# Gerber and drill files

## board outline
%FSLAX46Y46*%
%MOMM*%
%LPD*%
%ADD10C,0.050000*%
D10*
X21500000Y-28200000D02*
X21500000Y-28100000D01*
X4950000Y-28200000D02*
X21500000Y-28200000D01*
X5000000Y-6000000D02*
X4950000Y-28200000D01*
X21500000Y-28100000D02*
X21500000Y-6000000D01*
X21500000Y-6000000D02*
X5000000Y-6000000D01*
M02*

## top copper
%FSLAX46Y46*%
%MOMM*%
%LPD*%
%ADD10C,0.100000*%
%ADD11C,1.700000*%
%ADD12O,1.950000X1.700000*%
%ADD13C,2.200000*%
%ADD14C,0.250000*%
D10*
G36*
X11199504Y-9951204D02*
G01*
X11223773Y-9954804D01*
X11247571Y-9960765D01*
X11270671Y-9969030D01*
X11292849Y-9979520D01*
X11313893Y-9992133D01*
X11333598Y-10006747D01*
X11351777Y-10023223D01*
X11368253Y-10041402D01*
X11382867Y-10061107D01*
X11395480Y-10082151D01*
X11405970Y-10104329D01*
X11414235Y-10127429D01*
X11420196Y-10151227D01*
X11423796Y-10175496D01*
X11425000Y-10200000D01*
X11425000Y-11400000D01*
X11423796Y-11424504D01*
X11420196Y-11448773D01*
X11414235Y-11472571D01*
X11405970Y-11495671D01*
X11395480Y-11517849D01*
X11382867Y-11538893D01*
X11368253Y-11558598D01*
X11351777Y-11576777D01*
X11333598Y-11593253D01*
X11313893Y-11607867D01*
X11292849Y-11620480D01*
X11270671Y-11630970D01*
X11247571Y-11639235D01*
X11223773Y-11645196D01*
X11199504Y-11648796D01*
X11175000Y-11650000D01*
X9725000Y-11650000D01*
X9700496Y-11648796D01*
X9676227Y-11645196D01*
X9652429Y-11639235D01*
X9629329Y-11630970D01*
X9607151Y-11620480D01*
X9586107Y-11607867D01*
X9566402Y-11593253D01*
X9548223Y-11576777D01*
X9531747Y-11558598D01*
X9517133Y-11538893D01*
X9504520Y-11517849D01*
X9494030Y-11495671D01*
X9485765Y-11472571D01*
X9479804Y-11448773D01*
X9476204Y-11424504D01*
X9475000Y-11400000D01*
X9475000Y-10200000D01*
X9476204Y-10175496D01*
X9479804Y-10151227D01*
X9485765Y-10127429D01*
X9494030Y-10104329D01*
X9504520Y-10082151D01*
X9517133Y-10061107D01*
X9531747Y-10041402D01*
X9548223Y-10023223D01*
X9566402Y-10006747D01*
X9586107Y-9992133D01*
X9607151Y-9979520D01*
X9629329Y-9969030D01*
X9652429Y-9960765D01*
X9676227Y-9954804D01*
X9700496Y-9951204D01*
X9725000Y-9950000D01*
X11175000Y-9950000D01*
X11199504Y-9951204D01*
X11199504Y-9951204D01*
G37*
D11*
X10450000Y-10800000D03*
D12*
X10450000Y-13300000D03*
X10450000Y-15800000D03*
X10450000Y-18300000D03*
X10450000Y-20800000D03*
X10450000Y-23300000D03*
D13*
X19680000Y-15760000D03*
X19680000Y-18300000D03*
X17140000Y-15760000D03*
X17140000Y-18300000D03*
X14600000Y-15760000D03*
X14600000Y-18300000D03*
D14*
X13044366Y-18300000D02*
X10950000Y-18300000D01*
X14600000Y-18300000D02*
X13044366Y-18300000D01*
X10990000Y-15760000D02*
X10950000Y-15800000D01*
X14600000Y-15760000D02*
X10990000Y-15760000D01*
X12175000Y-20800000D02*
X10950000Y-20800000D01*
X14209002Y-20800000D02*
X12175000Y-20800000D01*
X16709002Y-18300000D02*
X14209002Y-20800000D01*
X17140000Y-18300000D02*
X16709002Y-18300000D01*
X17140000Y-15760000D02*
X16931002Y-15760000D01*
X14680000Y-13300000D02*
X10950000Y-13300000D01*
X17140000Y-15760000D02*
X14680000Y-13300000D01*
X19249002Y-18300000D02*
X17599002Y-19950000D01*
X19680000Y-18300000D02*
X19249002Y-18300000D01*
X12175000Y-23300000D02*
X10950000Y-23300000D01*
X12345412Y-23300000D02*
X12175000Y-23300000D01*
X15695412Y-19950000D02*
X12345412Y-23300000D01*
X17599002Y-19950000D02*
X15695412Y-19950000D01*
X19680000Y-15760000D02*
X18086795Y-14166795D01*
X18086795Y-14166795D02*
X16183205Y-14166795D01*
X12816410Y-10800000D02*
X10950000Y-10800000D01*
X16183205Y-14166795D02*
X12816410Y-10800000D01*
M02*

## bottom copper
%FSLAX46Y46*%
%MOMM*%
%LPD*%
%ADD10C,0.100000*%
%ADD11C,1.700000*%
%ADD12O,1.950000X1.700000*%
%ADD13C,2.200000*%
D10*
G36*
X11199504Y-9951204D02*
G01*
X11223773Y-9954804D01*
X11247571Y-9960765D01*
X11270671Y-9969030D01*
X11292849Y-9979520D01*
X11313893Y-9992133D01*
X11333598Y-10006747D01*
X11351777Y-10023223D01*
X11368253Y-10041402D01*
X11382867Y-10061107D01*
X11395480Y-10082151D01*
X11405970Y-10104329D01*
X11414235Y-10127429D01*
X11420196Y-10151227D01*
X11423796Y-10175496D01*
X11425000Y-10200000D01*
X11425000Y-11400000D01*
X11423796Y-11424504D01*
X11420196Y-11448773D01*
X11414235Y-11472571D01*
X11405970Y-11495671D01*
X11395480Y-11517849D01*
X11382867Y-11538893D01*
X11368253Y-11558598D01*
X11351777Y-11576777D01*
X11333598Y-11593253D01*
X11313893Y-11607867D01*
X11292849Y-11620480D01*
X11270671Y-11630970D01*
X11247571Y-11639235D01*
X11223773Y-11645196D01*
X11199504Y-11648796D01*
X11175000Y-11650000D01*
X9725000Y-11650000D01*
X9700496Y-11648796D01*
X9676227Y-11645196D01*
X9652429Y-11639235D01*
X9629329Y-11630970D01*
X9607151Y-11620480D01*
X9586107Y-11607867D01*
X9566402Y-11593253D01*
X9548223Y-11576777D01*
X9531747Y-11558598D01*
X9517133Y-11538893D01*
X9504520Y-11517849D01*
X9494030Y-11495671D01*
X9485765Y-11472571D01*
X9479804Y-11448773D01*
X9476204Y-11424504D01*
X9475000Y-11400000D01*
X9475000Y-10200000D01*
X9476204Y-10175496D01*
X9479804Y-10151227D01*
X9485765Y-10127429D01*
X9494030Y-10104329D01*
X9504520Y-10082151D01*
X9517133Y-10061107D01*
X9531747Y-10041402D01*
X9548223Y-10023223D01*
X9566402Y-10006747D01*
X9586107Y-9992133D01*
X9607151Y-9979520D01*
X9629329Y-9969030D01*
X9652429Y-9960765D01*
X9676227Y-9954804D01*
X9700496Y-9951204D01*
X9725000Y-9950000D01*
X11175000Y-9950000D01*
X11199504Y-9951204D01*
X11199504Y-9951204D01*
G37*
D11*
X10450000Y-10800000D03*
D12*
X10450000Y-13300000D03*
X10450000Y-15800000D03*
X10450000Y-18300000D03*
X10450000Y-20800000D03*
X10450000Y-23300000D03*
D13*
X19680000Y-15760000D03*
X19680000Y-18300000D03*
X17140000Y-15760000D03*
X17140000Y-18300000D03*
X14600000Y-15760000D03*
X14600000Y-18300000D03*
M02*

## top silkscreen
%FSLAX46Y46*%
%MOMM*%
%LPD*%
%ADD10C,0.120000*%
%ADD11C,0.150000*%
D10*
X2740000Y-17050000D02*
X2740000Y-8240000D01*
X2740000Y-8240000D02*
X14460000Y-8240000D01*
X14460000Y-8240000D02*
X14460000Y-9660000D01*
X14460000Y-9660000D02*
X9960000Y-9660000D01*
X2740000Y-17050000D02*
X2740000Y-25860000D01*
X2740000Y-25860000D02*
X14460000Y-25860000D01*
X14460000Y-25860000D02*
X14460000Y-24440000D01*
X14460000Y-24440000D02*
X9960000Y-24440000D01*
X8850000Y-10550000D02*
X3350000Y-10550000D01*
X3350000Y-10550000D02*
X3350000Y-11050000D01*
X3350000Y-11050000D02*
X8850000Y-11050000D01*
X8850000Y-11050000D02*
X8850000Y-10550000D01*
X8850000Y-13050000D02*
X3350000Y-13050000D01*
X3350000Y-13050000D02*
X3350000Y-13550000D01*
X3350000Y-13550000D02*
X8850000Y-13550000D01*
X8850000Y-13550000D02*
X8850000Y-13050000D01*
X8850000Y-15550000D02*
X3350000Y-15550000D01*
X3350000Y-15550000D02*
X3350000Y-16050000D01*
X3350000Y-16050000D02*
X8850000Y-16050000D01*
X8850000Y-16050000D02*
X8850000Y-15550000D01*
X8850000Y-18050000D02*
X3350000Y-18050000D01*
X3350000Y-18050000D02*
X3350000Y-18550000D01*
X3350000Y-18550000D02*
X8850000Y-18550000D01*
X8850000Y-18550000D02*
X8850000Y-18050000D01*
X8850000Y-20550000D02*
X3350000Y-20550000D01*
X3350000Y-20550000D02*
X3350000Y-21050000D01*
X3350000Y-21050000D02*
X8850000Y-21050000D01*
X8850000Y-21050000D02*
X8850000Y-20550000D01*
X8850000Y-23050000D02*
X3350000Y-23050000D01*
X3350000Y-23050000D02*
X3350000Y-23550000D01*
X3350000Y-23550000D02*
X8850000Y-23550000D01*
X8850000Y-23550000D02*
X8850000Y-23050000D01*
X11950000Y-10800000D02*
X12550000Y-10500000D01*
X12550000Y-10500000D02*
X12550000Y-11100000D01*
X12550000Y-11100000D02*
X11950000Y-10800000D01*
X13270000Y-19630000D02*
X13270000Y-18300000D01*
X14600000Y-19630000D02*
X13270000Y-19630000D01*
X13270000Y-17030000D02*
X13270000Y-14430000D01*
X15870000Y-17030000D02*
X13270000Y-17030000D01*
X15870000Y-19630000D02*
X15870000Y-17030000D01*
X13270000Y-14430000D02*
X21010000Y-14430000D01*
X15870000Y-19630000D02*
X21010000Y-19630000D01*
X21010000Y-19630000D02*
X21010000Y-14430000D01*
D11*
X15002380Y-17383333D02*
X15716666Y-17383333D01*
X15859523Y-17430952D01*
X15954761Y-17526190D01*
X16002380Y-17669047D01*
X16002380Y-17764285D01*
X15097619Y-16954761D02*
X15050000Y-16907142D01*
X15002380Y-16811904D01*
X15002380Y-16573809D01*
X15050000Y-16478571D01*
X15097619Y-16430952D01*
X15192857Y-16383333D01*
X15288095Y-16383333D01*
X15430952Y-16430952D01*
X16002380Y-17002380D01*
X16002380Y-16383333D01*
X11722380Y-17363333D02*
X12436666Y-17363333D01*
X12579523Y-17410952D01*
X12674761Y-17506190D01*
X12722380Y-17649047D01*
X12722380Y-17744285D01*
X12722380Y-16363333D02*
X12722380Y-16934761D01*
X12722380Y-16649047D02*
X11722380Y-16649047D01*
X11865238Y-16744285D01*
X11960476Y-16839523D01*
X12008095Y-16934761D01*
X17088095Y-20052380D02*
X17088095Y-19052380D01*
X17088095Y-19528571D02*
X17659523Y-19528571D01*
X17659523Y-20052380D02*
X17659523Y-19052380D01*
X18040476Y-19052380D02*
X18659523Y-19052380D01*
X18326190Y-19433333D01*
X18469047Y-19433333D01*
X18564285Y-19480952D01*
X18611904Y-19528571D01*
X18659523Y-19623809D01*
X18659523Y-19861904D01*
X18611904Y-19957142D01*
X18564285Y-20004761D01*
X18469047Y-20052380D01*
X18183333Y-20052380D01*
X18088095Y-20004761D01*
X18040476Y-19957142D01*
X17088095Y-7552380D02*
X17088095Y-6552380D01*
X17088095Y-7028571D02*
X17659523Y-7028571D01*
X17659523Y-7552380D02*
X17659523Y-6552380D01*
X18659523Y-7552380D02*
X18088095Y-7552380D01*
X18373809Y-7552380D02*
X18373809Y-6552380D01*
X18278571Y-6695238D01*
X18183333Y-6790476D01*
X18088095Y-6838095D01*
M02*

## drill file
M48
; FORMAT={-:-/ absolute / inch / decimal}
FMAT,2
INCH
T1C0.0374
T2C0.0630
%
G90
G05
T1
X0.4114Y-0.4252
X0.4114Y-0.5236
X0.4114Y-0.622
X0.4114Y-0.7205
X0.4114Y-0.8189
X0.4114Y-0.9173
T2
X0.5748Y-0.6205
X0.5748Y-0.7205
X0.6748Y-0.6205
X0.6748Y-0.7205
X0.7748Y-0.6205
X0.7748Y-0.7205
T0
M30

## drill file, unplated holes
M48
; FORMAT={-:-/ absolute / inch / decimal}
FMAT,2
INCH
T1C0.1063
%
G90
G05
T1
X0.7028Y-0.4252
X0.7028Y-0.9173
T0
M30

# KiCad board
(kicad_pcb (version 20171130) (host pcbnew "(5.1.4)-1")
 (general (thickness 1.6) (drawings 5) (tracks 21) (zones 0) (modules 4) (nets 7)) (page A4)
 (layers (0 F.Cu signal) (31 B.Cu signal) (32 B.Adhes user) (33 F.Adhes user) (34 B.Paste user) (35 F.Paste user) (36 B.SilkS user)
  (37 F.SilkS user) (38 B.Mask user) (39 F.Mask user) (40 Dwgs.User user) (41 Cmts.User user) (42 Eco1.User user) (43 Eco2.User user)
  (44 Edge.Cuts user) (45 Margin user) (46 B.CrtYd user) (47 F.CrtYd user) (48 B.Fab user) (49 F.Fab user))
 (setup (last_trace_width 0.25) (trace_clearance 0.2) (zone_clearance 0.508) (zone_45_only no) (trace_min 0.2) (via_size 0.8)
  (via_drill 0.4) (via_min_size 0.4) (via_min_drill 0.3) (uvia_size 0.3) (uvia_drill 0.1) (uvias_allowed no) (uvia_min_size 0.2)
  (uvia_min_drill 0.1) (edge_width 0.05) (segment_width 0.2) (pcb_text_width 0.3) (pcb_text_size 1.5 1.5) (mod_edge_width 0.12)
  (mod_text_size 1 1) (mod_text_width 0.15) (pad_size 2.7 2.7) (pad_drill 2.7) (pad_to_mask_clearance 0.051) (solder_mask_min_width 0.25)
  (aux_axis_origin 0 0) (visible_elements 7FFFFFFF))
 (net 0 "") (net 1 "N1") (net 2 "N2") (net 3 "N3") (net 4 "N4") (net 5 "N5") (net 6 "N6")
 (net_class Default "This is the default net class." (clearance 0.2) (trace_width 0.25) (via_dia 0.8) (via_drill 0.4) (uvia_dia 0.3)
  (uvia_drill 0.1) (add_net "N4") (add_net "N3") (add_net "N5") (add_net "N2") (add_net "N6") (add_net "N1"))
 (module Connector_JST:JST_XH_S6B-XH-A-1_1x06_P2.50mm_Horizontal (layer F.Cu) (at 10.45 10.8 270)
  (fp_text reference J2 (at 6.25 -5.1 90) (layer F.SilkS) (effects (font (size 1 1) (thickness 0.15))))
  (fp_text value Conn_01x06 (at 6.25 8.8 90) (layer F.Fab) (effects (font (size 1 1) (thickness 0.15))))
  (fp_line (start 6.25 7.71) (end -2.56 7.71) (layer F.SilkS) (width 0.12))
  (fp_line (start -2.56 7.71) (end -2.56 -4.01) (layer F.SilkS) (width 0.12))
  (fp_line (start -2.56 -4.01) (end -1.14 -4.01) (layer F.SilkS) (width 0.12))
  (fp_line (start -1.14 -4.01) (end -1.14 0.49) (layer F.SilkS) (width 0.12))
  (fp_line (start 6.25 7.71) (end 15.06 7.71) (layer F.SilkS) (width 0.12))
  (fp_line (start 15.06 7.71) (end 15.06 -4.01) (layer F.SilkS) (width 0.12))
  (fp_line (start 15.06 -4.01) (end 13.64 -4.01) (layer F.SilkS) (width 0.12))
  (fp_line (start 13.64 -4.01) (end 13.64 0.49) (layer F.SilkS) (width 0.12))
  (fp_line (start -0.25 1.6) (end -0.25 7.1) (layer F.SilkS) (width 0.12))
  (fp_line (start -0.25 7.1) (end 0.25 7.1) (layer F.SilkS) (width 0.12))
  (fp_line (start 0.25 7.1) (end 0.25 1.6) (layer F.SilkS) (width 0.12))
  (fp_line (start 0.25 1.6) (end -0.25 1.6) (layer F.SilkS) (width 0.12))
  (fp_line (start 2.25 1.6) (end 2.25 7.1) (layer F.SilkS) (width 0.12))
  (fp_line (start 2.25 7.1) (end 2.75 7.1) (layer F.SilkS) (width 0.12))
  (fp_line (start 2.75 7.1) (end 2.75 1.6) (layer F.SilkS) (width 0.12))
  (fp_line (start 2.75 1.6) (end 2.25 1.6) (layer F.SilkS) (width 0.12))
  (fp_line (start 4.75 1.6) (end 4.75 7.1) (layer F.SilkS) (width 0.12))
  (fp_line (start 4.75 7.1) (end 5.25 7.1) (layer F.SilkS) (width 0.12))
  (fp_line (start 5.25 7.1) (end 5.25 1.6) (layer F.SilkS) (width 0.12))
  (fp_line (start 5.25 1.6) (end 4.75 1.6) (layer F.SilkS) (width 0.12))
  (fp_line (start 7.25 1.6) (end 7.25 7.1) (layer F.SilkS) (width 0.12))
  (fp_line (start 7.25 7.1) (end 7.75 7.1) (layer F.SilkS) (width 0.12))
  (fp_line (start 7.75 7.1) (end 7.75 1.6) (layer F.SilkS) (width 0.12))
  (fp_line (start 7.75 1.6) (end 7.25 1.6) (layer F.SilkS) (width 0.12))
  (fp_line (start 9.75 1.6) (end 9.75 7.1) (layer F.SilkS) (width 0.12))
  (fp_line (start 9.75 7.1) (end 10.25 7.1) (layer F.SilkS) (width 0.12))
  (fp_line (start 10.25 7.1) (end 10.25 1.6) (layer F.SilkS) (width 0.12))
  (fp_line (start 10.25 1.6) (end 9.75 1.6) (layer F.SilkS) (width 0.12))
  (fp_line (start 12.25 1.6) (end 12.25 7.1) (layer F.SilkS) (width 0.12))
  (fp_line (start 12.25 7.1) (end 12.75 7.1) (layer F.SilkS) (width 0.12))
  (fp_line (start 12.75 7.1) (end 12.75 1.6) (layer F.SilkS) (width 0.12))
  (fp_line (start 12.75 1.6) (end 12.25 1.6) (layer F.SilkS) (width 0.12))
  (fp_line (start 0 -1.5) (end -0.3 -2.1) (layer F.SilkS) (width 0.12))
  (fp_line (start -0.3 -2.1) (end 0.3 -2.1) (layer F.SilkS) (width 0.12))
  (fp_line (start 0.3 -2.1) (end 0 -1.5) (layer F.SilkS) (width 0.12))
  (pad 1 thru_hole roundrect (at 0 0 270) (size 1.7 1.95) (drill 0.95) (layers *.Cu *.Mask) (roundrect_rratio 0.147059) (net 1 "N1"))
  (pad 2 thru_hole oval (at 2.5 0 270) (size 1.7 1.95) (drill 0.95) (layers *.Cu *.Mask) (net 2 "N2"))
  (pad 3 thru_hole oval (at 5 0 270) (size 1.7 1.95) (drill 0.95) (layers *.Cu *.Mask) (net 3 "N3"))
  (pad 4 thru_hole oval (at 7.5 0 270) (size 1.7 1.95) (drill 0.95) (layers *.Cu *.Mask) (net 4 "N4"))
  (pad 5 thru_hole oval (at 10 0 270) (size 1.7 1.95) (drill 0.95) (layers *.Cu *.Mask) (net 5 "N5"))
  (pad 6 thru_hole oval (at 12.5 0 270) (size 1.7 1.95) (drill 0.95) (layers *.Cu *.Mask) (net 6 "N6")))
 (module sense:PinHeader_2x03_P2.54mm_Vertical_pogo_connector (layer F.Cu) (at 14.6 18.3 90)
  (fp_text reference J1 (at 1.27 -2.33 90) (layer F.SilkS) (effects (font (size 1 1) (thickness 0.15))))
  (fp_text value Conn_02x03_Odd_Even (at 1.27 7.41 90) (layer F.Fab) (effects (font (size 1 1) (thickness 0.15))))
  (fp_line (start -1.33 -1.33) (end 0 -1.33) (layer F.SilkS) (width 0.12))
  (fp_line (start -1.33 0) (end -1.33 -1.33) (layer F.SilkS) (width 0.12))
  (fp_line (start 1.27 -1.33) (end 3.87 -1.33) (layer F.SilkS) (width 0.12))
  (fp_line (start 1.27 1.27) (end 1.27 -1.33) (layer F.SilkS) (width 0.12))
  (fp_line (start -1.33 1.27) (end 1.27 1.27) (layer F.SilkS) (width 0.12))
  (fp_line (start 3.87 -1.33) (end 3.87 6.41) (layer F.SilkS) (width 0.12))
  (fp_line (start -1.33 1.27) (end -1.33 6.41) (layer F.SilkS) (width 0.12))
  (fp_line (start -1.33 6.41) (end 3.87 6.41) (layer F.SilkS) (width 0.12))
  (pad 6 thru_hole circle (at 2.54 5.08 90) (size 2.2 2.2) (drill 1.6) (layers *.Cu *.Mask) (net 1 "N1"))
  (pad 5 thru_hole circle (at 0 5.08 90) (size 2.2 2.2) (drill 1.6) (layers *.Cu *.Mask) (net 6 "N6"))
  (pad 4 thru_hole circle (at 2.54 2.54 90) (size 2.2 2.2) (drill 1.6) (layers *.Cu *.Mask) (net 2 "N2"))
  (pad 3 thru_hole circle (at 0 2.54 90) (size 2.2 2.2) (drill 1.6) (layers *.Cu *.Mask) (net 5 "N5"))
  (pad 2 thru_hole circle (at 2.54 0 90) (size 2.2 2.2) (drill 1.6) (layers *.Cu *.Mask) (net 3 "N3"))
  (pad 1 thru_hole circle (at 0 0 90) (size 2.2 2.2) (drill 1.6) (layers *.Cu *.Mask) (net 4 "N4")))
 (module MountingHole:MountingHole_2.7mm (layer F.Cu) (at 17.85 23.3)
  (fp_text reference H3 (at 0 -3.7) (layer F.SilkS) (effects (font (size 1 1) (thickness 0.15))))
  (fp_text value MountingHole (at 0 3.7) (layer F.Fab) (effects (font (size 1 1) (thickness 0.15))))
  (pad 1 np_thru_hole circle (at 0 0) (size 2.7 2.7) (drill 2.7) (layers *.Cu *.Mask)))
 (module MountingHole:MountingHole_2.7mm (layer F.Cu) (at 17.85 10.8)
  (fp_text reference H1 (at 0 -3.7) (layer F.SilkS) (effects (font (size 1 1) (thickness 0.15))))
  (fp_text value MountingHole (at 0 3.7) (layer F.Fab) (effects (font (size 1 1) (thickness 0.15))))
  (pad "" np_thru_hole circle (at 0 0) (size 2.7 2.7) (drill 2.7) (layers *.Cu *.Mask)))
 (gr_line (start 21.5 28.2) (end 21.5 28.1) (layer Edge.Cuts) (width 0.05))
 (gr_line (start 4.95 28.2) (end 21.5 28.2) (layer Edge.Cuts) (width 0.05))
 (gr_line (start 5 6) (end 4.95 28.2) (layer Edge.Cuts) (width 0.05))
 (gr_line (start 21.5 28.1) (end 21.5 6) (layer Edge.Cuts) (width 0.05))
 (gr_line (start 21.5 6) (end 5 6) (layer Edge.Cuts) (width 0.05))
 (segment (start 13.044366 18.3) (end 10.95 18.3) (width 0.25) (layer F.Cu) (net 4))
 (segment (start 14.6 18.3) (end 13.044366 18.3) (width 0.25) (layer F.Cu) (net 4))
 (segment (start 10.99 15.76) (end 10.95 15.8) (width 0.25) (layer F.Cu) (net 3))
 (segment (start 14.6 15.76) (end 10.99 15.76) (width 0.25) (layer F.Cu) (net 3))
 (segment (start 12.175 20.8) (end 10.95 20.8) (width 0.25) (layer F.Cu) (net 5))
 (segment (start 14.209002 20.8) (end 12.175 20.8) (width 0.25) (layer F.Cu) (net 5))
 (segment (start 16.709002 18.3) (end 14.209002 20.8) (width 0.25) (layer F.Cu) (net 5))
 (segment (start 17.14 18.3) (end 16.709002 18.3) (width 0.25) (layer F.Cu) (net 5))
 (segment (start 17.14 15.76) (end 16.931002 15.76) (width 0.25) (layer F.Cu) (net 2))
 (segment (start 14.68 13.3) (end 10.95 13.3) (width 0.25) (layer F.Cu) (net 2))
 (segment (start 17.14 15.76) (end 14.68 13.3) (width 0.25) (layer F.Cu) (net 2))
 (segment (start 19.249002 18.3) (end 17.599002 19.95) (width 0.25) (layer F.Cu) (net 6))
 (segment (start 19.68 18.3) (end 19.249002 18.3) (width 0.25) (layer F.Cu) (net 6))
 (segment (start 12.175 23.3) (end 10.95 23.3) (width 0.25) (layer F.Cu) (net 6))
 (segment (start 12.345412 23.3) (end 12.175 23.3) (width 0.25) (layer F.Cu) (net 6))
 (segment (start 15.695412 19.95) (end 12.345412 23.3) (width 0.25) (layer F.Cu) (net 6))
 (segment (start 17.599002 19.95) (end 15.695412 19.95) (width 0.25) (layer F.Cu) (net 6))
 (segment (start 19.68 15.76) (end 18.086795 14.166795) (width 0.25) (layer F.Cu) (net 1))
 (segment (start 18.086795 14.166795) (end 16.183205 14.166795) (width 0.25) (layer F.Cu) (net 1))
 (segment (start 12.81641 10.8) (end 10.95 10.8) (width 0.25) (layer F.Cu) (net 1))
 (segment (start 16.183205 14.166795) (end 12.81641 10.8) (width 0.25) (layer F.Cu) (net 1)))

